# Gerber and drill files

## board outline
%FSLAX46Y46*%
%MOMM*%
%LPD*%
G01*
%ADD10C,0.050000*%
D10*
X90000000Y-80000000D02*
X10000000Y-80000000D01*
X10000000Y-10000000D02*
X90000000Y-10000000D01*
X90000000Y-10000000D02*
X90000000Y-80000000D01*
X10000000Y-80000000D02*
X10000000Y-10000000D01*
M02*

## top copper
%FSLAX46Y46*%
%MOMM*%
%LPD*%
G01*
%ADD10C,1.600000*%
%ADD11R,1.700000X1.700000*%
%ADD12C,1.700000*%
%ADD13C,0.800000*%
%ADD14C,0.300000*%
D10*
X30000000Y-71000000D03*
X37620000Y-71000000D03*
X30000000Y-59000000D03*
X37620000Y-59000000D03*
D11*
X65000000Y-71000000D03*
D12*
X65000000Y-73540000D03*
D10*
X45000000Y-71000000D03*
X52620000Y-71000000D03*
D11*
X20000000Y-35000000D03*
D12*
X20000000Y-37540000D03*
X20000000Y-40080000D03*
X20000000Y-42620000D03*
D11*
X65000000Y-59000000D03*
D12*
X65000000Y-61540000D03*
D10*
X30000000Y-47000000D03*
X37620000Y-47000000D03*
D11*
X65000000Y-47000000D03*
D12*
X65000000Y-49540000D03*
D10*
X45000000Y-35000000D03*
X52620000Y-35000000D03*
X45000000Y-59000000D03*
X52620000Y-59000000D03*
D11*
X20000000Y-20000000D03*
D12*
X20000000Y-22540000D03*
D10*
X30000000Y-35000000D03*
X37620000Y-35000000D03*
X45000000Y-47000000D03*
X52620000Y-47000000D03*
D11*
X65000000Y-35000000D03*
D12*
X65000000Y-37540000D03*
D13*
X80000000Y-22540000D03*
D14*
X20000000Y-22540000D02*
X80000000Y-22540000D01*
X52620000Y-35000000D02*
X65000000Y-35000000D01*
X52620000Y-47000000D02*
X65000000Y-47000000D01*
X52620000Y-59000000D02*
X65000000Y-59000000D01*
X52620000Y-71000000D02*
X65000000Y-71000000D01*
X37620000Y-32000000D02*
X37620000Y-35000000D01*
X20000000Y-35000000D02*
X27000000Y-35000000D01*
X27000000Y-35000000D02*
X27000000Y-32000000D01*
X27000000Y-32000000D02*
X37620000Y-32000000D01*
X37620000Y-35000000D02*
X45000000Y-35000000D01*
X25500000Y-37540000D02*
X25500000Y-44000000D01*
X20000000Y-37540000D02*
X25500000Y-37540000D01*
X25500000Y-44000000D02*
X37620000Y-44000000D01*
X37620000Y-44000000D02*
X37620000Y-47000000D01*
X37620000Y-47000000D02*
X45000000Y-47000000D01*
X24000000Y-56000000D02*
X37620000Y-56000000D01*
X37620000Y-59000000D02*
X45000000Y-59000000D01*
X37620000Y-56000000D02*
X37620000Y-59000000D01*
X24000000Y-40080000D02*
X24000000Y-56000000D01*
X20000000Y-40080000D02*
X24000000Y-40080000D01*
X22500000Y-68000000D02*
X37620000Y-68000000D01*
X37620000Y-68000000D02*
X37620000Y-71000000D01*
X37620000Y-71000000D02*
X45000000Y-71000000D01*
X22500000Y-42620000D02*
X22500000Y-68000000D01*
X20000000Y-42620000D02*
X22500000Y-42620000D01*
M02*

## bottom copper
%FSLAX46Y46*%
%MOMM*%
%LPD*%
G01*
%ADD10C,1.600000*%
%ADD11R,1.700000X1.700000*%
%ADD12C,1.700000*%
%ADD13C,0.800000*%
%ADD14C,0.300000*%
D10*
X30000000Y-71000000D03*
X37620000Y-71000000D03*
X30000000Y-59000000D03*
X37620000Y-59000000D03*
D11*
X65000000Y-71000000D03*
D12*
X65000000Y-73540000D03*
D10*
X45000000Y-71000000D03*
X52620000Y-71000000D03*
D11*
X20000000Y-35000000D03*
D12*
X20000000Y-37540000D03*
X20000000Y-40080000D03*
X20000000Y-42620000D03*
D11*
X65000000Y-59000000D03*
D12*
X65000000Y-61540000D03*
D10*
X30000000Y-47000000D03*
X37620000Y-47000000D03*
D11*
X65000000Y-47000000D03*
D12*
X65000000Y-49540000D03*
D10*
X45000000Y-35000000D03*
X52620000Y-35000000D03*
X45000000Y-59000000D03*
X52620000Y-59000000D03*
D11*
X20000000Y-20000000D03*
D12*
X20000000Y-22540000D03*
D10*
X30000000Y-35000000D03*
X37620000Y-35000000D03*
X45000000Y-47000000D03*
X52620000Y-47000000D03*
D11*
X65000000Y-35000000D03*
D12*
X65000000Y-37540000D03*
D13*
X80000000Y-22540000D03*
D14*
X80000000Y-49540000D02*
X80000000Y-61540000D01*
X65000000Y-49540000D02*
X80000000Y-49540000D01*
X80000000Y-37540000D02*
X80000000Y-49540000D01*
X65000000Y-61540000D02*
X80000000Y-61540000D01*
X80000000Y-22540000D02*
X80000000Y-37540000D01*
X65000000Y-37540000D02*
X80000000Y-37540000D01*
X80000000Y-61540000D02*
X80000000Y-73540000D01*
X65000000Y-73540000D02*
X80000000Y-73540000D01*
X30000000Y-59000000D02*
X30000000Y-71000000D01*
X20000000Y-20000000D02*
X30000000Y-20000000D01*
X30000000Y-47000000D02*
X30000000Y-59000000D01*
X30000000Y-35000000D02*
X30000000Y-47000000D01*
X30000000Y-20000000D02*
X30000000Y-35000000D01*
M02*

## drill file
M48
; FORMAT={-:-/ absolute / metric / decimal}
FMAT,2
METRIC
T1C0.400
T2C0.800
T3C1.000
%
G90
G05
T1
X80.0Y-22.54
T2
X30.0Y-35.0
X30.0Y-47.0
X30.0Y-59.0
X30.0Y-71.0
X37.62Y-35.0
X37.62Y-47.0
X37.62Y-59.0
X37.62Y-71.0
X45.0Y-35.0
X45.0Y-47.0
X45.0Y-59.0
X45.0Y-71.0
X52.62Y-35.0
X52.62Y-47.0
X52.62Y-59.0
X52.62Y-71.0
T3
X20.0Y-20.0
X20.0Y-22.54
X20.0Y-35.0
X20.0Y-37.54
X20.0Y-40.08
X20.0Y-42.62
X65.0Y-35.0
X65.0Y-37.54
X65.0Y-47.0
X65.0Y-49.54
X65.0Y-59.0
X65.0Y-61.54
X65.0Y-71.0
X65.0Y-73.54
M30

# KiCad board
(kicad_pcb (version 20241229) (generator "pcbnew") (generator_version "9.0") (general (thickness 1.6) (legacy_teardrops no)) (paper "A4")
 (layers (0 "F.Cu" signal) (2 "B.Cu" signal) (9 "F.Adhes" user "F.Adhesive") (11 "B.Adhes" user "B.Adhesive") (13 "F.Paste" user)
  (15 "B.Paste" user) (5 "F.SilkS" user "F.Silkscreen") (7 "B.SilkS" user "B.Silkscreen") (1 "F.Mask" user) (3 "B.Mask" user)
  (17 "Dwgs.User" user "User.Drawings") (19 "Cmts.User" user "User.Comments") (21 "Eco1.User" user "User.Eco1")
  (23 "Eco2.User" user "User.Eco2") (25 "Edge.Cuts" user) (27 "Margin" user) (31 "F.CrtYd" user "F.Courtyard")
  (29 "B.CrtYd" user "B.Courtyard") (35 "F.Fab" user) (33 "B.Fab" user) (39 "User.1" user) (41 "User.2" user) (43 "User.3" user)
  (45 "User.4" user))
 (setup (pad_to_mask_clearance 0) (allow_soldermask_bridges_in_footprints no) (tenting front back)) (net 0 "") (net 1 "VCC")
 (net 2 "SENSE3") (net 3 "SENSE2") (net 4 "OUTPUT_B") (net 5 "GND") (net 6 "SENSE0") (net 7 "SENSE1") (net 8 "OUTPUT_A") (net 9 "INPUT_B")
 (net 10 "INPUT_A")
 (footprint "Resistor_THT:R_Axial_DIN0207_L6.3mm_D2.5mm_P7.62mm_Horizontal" (layer "F.Cu") (at 30 71)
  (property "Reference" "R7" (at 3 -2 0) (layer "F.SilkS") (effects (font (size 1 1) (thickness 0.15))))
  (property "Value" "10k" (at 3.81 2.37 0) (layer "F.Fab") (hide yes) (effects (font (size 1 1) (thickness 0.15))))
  (pad "1" thru_hole circle (at 0 0) (size 1.6 1.6) (drill 0.8) (layers "*.Cu" "*.Mask") (remove_unused_layers no) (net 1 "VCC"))
  (pad "2" thru_hole circle (at 7.62 0) (size 1.6 1.6) (drill 0.8) (layers "*.Cu" "*.Mask") (remove_unused_layers no) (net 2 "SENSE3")))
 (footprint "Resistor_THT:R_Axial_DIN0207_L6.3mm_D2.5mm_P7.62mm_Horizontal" (layer "F.Cu") (at 30 59)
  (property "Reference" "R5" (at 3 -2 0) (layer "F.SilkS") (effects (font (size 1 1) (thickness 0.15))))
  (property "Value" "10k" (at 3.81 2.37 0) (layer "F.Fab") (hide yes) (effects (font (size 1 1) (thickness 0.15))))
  (pad "1" thru_hole circle (at 0 0) (size 1.6 1.6) (drill 0.8) (layers "*.Cu" "*.Mask") (remove_unused_layers no) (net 1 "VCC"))
  (pad "2" thru_hole circle (at 7.62 0) (size 1.6 1.6) (drill 0.8) (layers "*.Cu" "*.Mask") (remove_unused_layers no) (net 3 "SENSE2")))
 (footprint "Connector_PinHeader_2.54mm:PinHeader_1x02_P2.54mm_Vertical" (layer "F.Cu") (at 65 71)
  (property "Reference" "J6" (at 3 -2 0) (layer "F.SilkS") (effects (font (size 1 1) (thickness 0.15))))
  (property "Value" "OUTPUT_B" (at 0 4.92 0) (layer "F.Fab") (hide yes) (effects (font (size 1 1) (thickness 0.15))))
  (pad "1" thru_hole rect (at 0 0) (size 1.7 1.7) (drill 1) (layers "*.Cu" "*.Mask") (remove_unused_layers no) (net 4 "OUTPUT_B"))
  (pad "2" thru_hole circle (at 0 2.54) (size 1.7 1.7) (drill 1) (layers "*.Cu" "*.Mask") (remove_unused_layers no) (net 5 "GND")))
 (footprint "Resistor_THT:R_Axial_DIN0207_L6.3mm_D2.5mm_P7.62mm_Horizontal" (layer "F.Cu") (at 45 71)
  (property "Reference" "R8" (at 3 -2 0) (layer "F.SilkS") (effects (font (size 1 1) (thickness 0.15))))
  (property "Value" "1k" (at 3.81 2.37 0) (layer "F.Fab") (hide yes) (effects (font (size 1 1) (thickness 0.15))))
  (pad "1" thru_hole circle (at 0 0) (size 1.6 1.6) (drill 0.8) (layers "*.Cu" "*.Mask") (remove_unused_layers no) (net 2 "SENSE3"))
  (pad "2" thru_hole circle (at 7.62 0) (size 1.6 1.6) (drill 0.8) (layers "*.Cu" "*.Mask") (remove_unused_layers no) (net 4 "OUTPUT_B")))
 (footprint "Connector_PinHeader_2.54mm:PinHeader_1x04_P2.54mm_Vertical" (layer "F.Cu") (at 20 35)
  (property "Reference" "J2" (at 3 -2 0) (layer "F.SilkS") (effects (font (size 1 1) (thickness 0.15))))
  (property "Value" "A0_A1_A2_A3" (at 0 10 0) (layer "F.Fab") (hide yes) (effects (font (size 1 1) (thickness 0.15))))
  (pad "1" thru_hole rect (at 0 0) (size 1.7 1.7) (drill 1) (layers "*.Cu" "*.Mask") (remove_unused_layers no) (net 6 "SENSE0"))
  (pad "2" thru_hole circle (at 0 2.54) (size 1.7 1.7) (drill 1) (layers "*.Cu" "*.Mask") (remove_unused_layers no) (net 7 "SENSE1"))
  (pad "3" thru_hole circle (at 0 5.08) (size 1.7 1.7) (drill 1) (layers "*.Cu" "*.Mask") (remove_unused_layers no) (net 3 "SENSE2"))
  (pad "4" thru_hole circle (at 0 7.62) (size 1.7 1.7) (drill 1) (layers "*.Cu" "*.Mask") (remove_unused_layers no) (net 2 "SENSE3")))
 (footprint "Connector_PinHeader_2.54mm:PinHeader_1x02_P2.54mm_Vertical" (layer "F.Cu") (at 65 59)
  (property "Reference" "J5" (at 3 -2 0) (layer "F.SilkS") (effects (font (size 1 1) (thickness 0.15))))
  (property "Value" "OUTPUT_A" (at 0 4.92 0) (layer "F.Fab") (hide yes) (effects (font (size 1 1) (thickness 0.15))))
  (pad "1" thru_hole rect (at 0 0) (size 1.7 1.7) (drill 1) (layers "*.Cu" "*.Mask") (remove_unused_layers no) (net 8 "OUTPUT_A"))
  (pad "2" thru_hole circle (at 0 2.54) (size 1.7 1.7) (drill 1) (layers "*.Cu" "*.Mask") (remove_unused_layers no) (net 5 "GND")))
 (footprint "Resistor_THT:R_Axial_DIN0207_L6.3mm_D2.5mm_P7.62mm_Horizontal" (layer "F.Cu") (at 30 47)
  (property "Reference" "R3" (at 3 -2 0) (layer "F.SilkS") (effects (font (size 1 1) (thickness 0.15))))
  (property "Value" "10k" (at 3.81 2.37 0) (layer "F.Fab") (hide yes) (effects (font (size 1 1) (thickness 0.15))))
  (pad "1" thru_hole circle (at 0 0) (size 1.6 1.6) (drill 0.8) (layers "*.Cu" "*.Mask") (remove_unused_layers no) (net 1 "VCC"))
  (pad "2" thru_hole circle (at 7.62 0) (size 1.6 1.6) (drill 0.8) (layers "*.Cu" "*.Mask") (remove_unused_layers no) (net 7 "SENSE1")))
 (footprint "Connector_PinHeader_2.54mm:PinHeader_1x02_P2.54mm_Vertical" (layer "F.Cu") (at 65 47)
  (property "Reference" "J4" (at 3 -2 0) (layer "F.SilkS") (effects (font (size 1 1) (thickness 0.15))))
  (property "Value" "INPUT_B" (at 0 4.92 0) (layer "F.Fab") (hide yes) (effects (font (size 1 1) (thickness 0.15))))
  (pad "1" thru_hole rect (at 0 0) (size 1.7 1.7) (drill 1) (layers "*.Cu" "*.Mask") (remove_unused_layers no) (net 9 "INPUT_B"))
  (pad "2" thru_hole circle (at 0 2.54) (size 1.7 1.7) (drill 1) (layers "*.Cu" "*.Mask") (remove_unused_layers no) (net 5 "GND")))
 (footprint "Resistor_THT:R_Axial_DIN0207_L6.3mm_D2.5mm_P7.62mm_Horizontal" (layer "F.Cu") (at 45 35)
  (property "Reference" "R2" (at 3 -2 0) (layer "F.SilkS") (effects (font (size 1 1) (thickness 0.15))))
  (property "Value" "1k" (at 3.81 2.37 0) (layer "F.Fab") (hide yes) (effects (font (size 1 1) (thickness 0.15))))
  (pad "1" thru_hole circle (at 0 0) (size 1.6 1.6) (drill 0.8) (layers "*.Cu" "*.Mask") (remove_unused_layers no) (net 6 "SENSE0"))
  (pad "2" thru_hole circle (at 7.62 0) (size 1.6 1.6) (drill 0.8) (layers "*.Cu" "*.Mask") (remove_unused_layers no) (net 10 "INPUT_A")))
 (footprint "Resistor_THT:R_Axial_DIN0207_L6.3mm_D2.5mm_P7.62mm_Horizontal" (layer "F.Cu") (at 45 59)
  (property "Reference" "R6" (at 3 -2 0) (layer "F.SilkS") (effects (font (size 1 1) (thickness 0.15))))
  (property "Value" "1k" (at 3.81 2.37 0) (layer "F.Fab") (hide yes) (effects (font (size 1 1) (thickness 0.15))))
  (pad "1" thru_hole circle (at 0 0) (size 1.6 1.6) (drill 0.8) (layers "*.Cu" "*.Mask") (remove_unused_layers no) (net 3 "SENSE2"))
  (pad "2" thru_hole circle (at 7.62 0) (size 1.6 1.6) (drill 0.8) (layers "*.Cu" "*.Mask") (remove_unused_layers no) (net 8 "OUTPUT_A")))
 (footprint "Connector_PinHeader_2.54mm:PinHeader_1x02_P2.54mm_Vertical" (layer "F.Cu") (at 20 20)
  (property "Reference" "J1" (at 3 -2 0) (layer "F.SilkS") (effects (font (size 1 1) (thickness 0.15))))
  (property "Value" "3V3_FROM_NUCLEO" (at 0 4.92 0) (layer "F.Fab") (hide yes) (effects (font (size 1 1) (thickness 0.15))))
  (pad "1" thru_hole rect (at 0 0) (size 1.7 1.7) (drill 1) (layers "*.Cu" "*.Mask") (remove_unused_layers no) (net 1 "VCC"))
  (pad "2" thru_hole circle (at 0 2.54) (size 1.7 1.7) (drill 1) (layers "*.Cu" "*.Mask") (remove_unused_layers no) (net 5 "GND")))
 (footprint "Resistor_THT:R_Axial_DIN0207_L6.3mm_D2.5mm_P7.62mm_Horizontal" (layer "F.Cu") (at 30 35)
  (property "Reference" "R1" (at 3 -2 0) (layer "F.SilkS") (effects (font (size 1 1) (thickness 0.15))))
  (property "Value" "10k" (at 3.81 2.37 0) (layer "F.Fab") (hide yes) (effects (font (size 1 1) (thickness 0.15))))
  (pad "1" thru_hole circle (at 0 0) (size 1.6 1.6) (drill 0.8) (layers "*.Cu" "*.Mask") (remove_unused_layers no) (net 1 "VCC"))
  (pad "2" thru_hole circle (at 7.62 0) (size 1.6 1.6) (drill 0.8) (layers "*.Cu" "*.Mask") (remove_unused_layers no) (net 6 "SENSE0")))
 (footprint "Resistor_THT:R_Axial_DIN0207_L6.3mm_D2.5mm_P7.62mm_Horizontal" (layer "F.Cu") (at 45 47)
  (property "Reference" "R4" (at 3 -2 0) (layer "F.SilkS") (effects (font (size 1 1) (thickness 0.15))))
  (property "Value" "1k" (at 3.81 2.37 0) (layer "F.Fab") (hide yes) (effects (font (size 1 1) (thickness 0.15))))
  (pad "1" thru_hole circle (at 0 0) (size 1.6 1.6) (drill 0.8) (layers "*.Cu" "*.Mask") (remove_unused_layers no) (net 7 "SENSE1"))
  (pad "2" thru_hole circle (at 7.62 0) (size 1.6 1.6) (drill 0.8) (layers "*.Cu" "*.Mask") (remove_unused_layers no) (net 9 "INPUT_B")))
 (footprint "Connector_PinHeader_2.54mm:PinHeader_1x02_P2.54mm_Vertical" (layer "F.Cu") (at 65 35)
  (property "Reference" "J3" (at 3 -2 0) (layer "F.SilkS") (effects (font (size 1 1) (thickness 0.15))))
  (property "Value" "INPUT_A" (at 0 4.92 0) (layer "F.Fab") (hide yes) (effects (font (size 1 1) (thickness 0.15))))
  (pad "1" thru_hole rect (at 0 0) (size 1.7 1.7) (drill 1) (layers "*.Cu" "*.Mask") (remove_unused_layers no) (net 10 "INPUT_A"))
  (pad "2" thru_hole circle (at 0 2.54) (size 1.7 1.7) (drill 1) (layers "*.Cu" "*.Mask") (remove_unused_layers no) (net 5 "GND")))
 (gr_line (start 90 80) (end 10 80) (stroke (width 0.05) (type default)) (layer "Edge.Cuts"))
 (gr_line (start 10 10) (end 90 10) (stroke (width 0.05) (type default)) (layer "Edge.Cuts"))
 (gr_line (start 90 10) (end 90 80) (stroke (width 0.05) (type default)) (layer "Edge.Cuts"))
 (gr_line (start 10 80) (end 10 10) (stroke (width 0.05) (type default)) (layer "Edge.Cuts"))
 (segment (start 20 22.54) (end 80 22.54) (width 0.3) (layer "F.Cu") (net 5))
 (via (at 80 22.54) (size 0.8) (drill 0.4) (layers "F.Cu" "B.Cu") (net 5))
 (segment (start 80 49.54) (end 80 61.54) (width 0.3) (layer "B.Cu") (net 5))
 (segment (start 65 49.54) (end 80 49.54) (width 0.3) (layer "B.Cu") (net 5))
 (segment (start 80 37.54) (end 80 49.54) (width 0.3) (layer "B.Cu") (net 5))
 (segment (start 65 61.54) (end 80 61.54) (width 0.3) (layer "B.Cu") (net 5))
 (segment (start 80 22.54) (end 80 37.54) (width 0.3) (layer "B.Cu") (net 5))
 (segment (start 65 37.54) (end 80 37.54) (width 0.3) (layer "B.Cu") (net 5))
 (segment (start 80 61.54) (end 80 73.54) (width 0.3) (layer "B.Cu") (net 5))
 (segment (start 65 73.54) (end 80 73.54) (width 0.3) (layer "B.Cu") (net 5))
 (segment (start 52.62 35) (end 65 35) (width 0.3) (layer "F.Cu") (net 10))
 (segment (start 52.62 47) (end 65 47) (width 0.3) (layer "F.Cu") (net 9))
 (segment (start 52.62 59) (end 65 59) (width 0.3) (layer "F.Cu") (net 8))
 (segment (start 52.62 71) (end 65 71) (width 0.3) (layer "F.Cu") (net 4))
 (segment (start 37.62 32) (end 37.62 35) (width 0.3) (layer "F.Cu") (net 6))
 (segment (start 20 35) (end 27 35) (width 0.3) (layer "F.Cu") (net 6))
 (segment (start 27 35) (end 27 32) (width 0.3) (layer "F.Cu") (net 6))
 (segment (start 27 32) (end 37.62 32) (width 0.3) (layer "F.Cu") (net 6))
 (segment (start 37.62 35) (end 45 35) (width 0.3) (layer "F.Cu") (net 6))
 (segment (start 25.5 37.54) (end 25.5 44) (width 0.3) (layer "F.Cu") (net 7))
 (segment (start 20 37.54) (end 25.5 37.54) (width 0.3) (layer "F.Cu") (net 7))
 (segment (start 25.5 44) (end 37.62 44) (width 0.3) (layer "F.Cu") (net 7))
 (segment (start 37.62 44) (end 37.62 47) (width 0.3) (layer "F.Cu") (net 7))
 (segment (start 37.62 47) (end 45 47) (width 0.3) (layer "F.Cu") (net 7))
 (segment (start 24 56) (end 37.62 56) (width 0.3) (layer "F.Cu") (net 3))
 (segment (start 37.62 59) (end 45 59) (width 0.3) (layer "F.Cu") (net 3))
 (segment (start 37.62 56) (end 37.62 59) (width 0.3) (layer "F.Cu") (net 3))
 (segment (start 24 40.08) (end 24 56) (width 0.3) (layer "F.Cu") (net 3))
 (segment (start 20 40.08) (end 24 40.08) (width 0.3) (layer "F.Cu") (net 3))
 (segment (start 22.5 68) (end 37.62 68) (width 0.3) (layer "F.Cu") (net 2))
 (segment (start 37.62 68) (end 37.62 71) (width 0.3) (layer "F.Cu") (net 2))
 (segment (start 37.62 71) (end 45 71) (width 0.3) (layer "F.Cu") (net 2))
 (segment (start 22.5 42.62) (end 22.5 68) (width 0.3) (layer "F.Cu") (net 2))
 (segment (start 20 42.62) (end 22.5 42.62) (width 0.3) (layer "F.Cu") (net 2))
 (segment (start 30 59) (end 30 71) (width 0.3) (layer "B.Cu") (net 1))
 (segment (start 20 20) (end 30 20) (width 0.3) (layer "B.Cu") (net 1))
 (segment (start 30 47) (end 30 59) (width 0.3) (layer "B.Cu") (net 1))
 (segment (start 30 35) (end 30 47) (width 0.3) (layer "B.Cu") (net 1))
 (segment (start 30 20) (end 30 35) (width 0.3) (layer "B.Cu") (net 1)))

